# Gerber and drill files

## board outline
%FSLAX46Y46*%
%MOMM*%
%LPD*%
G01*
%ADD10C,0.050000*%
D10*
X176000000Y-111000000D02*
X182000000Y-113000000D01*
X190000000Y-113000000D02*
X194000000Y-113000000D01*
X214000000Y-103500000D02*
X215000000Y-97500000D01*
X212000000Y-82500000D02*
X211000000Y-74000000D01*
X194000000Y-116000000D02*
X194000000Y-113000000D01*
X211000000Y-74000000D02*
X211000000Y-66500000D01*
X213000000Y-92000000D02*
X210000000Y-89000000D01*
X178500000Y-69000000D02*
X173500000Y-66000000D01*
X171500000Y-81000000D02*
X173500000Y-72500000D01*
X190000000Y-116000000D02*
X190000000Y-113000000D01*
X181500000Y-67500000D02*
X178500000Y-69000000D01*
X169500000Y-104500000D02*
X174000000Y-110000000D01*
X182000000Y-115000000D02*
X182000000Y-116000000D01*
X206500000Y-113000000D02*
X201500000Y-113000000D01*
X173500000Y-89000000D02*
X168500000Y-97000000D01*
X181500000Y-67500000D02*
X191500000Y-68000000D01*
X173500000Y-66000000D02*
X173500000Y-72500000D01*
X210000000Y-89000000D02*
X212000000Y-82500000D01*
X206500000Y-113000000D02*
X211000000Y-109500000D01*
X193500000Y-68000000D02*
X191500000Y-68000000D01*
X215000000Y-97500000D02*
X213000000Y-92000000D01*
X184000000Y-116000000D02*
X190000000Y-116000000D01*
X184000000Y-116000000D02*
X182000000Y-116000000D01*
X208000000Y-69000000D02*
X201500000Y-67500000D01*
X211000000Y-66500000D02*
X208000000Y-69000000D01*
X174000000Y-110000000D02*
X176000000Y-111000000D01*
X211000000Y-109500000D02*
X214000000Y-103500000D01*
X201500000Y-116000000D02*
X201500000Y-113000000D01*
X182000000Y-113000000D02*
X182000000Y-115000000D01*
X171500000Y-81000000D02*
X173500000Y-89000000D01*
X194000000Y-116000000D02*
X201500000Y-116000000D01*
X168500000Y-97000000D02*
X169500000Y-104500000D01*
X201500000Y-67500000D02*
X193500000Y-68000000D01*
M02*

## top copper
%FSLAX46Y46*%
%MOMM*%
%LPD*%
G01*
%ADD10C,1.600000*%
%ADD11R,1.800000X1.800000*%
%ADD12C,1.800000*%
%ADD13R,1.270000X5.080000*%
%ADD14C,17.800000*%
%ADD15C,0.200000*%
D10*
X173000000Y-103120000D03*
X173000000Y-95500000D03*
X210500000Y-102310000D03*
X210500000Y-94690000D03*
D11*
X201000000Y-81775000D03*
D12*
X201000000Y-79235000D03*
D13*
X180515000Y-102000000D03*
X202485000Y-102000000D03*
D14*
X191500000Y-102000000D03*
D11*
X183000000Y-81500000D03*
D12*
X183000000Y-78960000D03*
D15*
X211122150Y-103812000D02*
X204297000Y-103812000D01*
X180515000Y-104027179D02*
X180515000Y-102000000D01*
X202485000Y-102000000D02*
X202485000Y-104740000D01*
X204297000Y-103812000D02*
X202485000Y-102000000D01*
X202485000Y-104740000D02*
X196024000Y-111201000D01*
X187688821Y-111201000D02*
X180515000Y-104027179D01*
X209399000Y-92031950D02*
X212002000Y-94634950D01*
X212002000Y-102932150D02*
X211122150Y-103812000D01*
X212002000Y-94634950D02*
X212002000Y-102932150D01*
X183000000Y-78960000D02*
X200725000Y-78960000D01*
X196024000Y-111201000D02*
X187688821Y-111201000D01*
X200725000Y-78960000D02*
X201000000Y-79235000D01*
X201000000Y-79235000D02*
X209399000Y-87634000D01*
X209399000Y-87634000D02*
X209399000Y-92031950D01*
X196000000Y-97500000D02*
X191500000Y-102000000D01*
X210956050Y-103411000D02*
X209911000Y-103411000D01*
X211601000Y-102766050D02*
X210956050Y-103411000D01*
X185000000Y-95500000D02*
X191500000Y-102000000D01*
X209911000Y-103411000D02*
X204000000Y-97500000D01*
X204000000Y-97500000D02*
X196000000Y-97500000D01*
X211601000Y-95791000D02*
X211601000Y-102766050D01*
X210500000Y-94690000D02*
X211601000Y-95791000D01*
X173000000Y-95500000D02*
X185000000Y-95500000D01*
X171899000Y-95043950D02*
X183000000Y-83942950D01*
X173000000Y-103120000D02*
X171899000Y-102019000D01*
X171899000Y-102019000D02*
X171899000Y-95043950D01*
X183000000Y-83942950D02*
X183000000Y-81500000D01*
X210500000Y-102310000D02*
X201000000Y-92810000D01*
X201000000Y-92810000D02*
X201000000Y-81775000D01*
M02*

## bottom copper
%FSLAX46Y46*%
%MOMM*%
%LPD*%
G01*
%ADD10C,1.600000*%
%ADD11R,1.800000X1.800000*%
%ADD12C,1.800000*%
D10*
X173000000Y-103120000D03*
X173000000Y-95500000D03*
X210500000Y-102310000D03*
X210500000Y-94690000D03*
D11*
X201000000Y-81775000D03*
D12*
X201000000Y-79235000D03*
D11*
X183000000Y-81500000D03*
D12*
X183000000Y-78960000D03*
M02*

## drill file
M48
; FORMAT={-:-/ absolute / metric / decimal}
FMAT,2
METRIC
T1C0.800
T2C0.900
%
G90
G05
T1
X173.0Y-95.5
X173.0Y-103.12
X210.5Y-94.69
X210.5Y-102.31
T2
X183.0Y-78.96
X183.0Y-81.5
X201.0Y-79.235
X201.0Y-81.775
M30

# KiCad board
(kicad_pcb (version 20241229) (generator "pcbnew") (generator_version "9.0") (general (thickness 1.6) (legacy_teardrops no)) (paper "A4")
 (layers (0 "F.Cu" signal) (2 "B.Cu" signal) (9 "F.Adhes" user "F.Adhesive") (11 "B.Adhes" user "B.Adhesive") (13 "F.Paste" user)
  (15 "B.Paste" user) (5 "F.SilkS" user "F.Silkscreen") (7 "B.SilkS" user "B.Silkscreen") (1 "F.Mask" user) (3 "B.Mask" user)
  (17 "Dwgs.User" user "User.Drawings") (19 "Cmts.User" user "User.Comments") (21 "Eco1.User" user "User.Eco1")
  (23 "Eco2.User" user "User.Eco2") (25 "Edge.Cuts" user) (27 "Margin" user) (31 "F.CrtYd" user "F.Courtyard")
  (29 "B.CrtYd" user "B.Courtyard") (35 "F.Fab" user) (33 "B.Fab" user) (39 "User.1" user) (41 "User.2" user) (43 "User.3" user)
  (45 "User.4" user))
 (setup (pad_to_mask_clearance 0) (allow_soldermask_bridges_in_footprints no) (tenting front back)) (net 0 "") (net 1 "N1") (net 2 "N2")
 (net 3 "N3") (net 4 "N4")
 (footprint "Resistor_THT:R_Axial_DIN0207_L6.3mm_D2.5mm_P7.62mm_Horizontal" (layer "F.Cu") (at 173 103.12 90)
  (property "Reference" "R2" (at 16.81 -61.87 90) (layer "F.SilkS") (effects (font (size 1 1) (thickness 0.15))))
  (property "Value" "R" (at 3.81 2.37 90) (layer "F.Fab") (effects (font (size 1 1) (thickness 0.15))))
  (pad "1" thru_hole circle (at 0 0 90) (size 1.6 1.6) (drill 0.8) (layers "*.Cu" "*.Mask") (remove_unused_layers no) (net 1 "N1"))
  (pad "2" thru_hole circle (at 7.62 0 90) (size 1.6 1.6) (drill 0.8) (layers "*.Cu" "*.Mask") (remove_unused_layers no) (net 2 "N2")))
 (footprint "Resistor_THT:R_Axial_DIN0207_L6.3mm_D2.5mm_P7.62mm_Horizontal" (layer "F.Cu") (at 210.5 102.31 90)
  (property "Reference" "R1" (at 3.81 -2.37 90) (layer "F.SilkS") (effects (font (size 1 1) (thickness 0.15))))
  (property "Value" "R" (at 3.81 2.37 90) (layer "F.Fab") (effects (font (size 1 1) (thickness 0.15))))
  (pad "1" thru_hole circle (at 0 0 90) (size 1.6 1.6) (drill 0.8) (layers "*.Cu" "*.Mask") (remove_unused_layers no) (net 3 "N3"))
  (pad "2" thru_hole circle (at 7.62 0 90) (size 1.6 1.6) (drill 0.8) (layers "*.Cu" "*.Mask") (remove_unused_layers no) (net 2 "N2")))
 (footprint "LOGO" (layer "F.Cu") (at 192 79)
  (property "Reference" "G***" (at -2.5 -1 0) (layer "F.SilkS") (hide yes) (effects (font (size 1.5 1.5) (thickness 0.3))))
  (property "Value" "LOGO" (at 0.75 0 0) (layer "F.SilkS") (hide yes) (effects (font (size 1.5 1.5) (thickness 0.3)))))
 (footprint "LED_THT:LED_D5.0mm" (layer "F.Cu") (at 201 81.775 90)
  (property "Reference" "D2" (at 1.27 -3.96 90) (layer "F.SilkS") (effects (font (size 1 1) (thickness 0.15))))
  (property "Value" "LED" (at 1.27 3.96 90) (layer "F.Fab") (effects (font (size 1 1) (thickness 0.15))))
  (pad "1" thru_hole rect (at 0 0 90) (size 1.8 1.8) (drill 0.9) (layers "*.Cu" "*.Mask") (remove_unused_layers no) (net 3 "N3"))
  (pad "2" thru_hole circle (at 2.54 0 90) (size 1.8 1.8) (drill 0.9) (layers "*.Cu" "*.Mask") (remove_unused_layers no) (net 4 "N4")))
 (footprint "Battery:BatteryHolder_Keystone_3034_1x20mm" (layer "F.Cu") (at 191.5 102)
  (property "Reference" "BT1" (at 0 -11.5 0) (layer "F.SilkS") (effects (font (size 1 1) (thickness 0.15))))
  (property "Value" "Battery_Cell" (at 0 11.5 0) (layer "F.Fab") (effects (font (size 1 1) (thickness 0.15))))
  (pad "1" smd rect (at -10.985 0) (size 1.27 5.08) (layers "F.Cu" "F.Mask" "F.Paste") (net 4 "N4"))
  (pad "1" smd rect (at 10.985 0) (size 1.27 5.08) (layers "F.Cu" "F.Mask" "F.Paste") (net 4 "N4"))
  (pad "2" smd circle (at 0 0) (size 17.8 17.8) (layers "F.Cu" "F.Mask") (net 2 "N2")))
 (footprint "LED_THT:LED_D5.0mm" (layer "F.Cu") (at 183 81.5 90)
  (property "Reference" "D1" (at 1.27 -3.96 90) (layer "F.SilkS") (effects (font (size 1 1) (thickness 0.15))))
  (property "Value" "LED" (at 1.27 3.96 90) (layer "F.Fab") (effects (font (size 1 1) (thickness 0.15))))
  (pad "1" thru_hole rect (at 0 0 90) (size 1.8 1.8) (drill 0.9) (layers "*.Cu" "*.Mask") (remove_unused_layers no) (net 1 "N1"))
  (pad "2" thru_hole circle (at 2.54 0 90) (size 1.8 1.8) (drill 0.9) (layers "*.Cu" "*.Mask") (remove_unused_layers no) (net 4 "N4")))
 (gr_line (start 176 111) (end 182 113) (stroke (width 0.05) (type default)) (layer "Edge.Cuts"))
 (gr_line (start 190 113) (end 194 113) (stroke (width 0.05) (type default)) (layer "Edge.Cuts"))
 (gr_line (start 214 103.5) (end 215 97.5) (stroke (width 0.05) (type default)) (layer "Edge.Cuts"))
 (gr_line (start 212 82.5) (end 211 74) (stroke (width 0.05) (type default)) (layer "Edge.Cuts"))
 (gr_line (start 194 116) (end 194 113) (stroke (width 0.05) (type default)) (layer "Edge.Cuts"))
 (gr_line (start 211 74) (end 211 66.5) (stroke (width 0.05) (type default)) (layer "Edge.Cuts"))
 (gr_line (start 213 92) (end 210 89) (stroke (width 0.05) (type default)) (layer "Edge.Cuts"))
 (gr_line (start 178.5 69) (end 173.5 66) (stroke (width 0.05) (type default)) (layer "Edge.Cuts"))
 (gr_line (start 171.5 81) (end 173.5 72.5) (stroke (width 0.05) (type default)) (layer "Edge.Cuts"))
 (gr_line (start 190 116) (end 190 113) (stroke (width 0.05) (type default)) (layer "Edge.Cuts"))
 (gr_line (start 181.5 67.5) (end 178.5 69) (stroke (width 0.05) (type default)) (layer "Edge.Cuts"))
 (gr_line (start 169.5 104.5) (end 174 110) (stroke (width 0.05) (type default)) (layer "Edge.Cuts"))
 (gr_line (start 182 115) (end 182 116) (stroke (width 0.05) (type default)) (layer "Edge.Cuts"))
 (gr_line (start 206.5 113) (end 201.5 113) (stroke (width 0.05) (type default)) (layer "Edge.Cuts"))
 (gr_line (start 173.5 89) (end 168.5 97) (stroke (width 0.05) (type default)) (layer "Edge.Cuts"))
 (gr_line (start 181.5 67.5) (end 191.5 68) (stroke (width 0.05) (type default)) (layer "Edge.Cuts"))
 (gr_line (start 173.5 66) (end 173.5 72.5) (stroke (width 0.05) (type default)) (layer "Edge.Cuts"))
 (gr_line (start 210 89) (end 212 82.5) (stroke (width 0.05) (type default)) (layer "Edge.Cuts"))
 (gr_line (start 206.5 113) (end 211 109.5) (stroke (width 0.05) (type default)) (layer "Edge.Cuts"))
 (gr_line (start 193.5 68) (end 191.5 68) (stroke (width 0.05) (type default)) (layer "Edge.Cuts"))
 (gr_line (start 215 97.5) (end 213 92) (stroke (width 0.05) (type default)) (layer "Edge.Cuts"))
 (gr_line (start 184 116) (end 190 116) (stroke (width 0.05) (type default)) (layer "Edge.Cuts"))
 (gr_line (start 184 116) (end 182 116) (stroke (width 0.05) (type default)) (layer "Edge.Cuts"))
 (gr_line (start 208 69) (end 201.5 67.5) (stroke (width 0.05) (type default)) (layer "Edge.Cuts"))
 (gr_line (start 211 66.5) (end 208 69) (stroke (width 0.05) (type default)) (layer "Edge.Cuts"))
 (gr_line (start 174 110) (end 176 111) (stroke (width 0.05) (type default)) (layer "Edge.Cuts"))
 (gr_line (start 211 109.5) (end 214 103.5) (stroke (width 0.05) (type default)) (layer "Edge.Cuts"))
 (gr_line (start 201.5 116) (end 201.5 113) (stroke (width 0.05) (type default)) (layer "Edge.Cuts"))
 (gr_line (start 182 113) (end 182 115) (stroke (width 0.05) (type default)) (layer "Edge.Cuts"))
 (gr_line (start 171.5 81) (end 173.5 89) (stroke (width 0.05) (type default)) (layer "Edge.Cuts"))
 (gr_line (start 194 116) (end 201.5 116) (stroke (width 0.05) (type default)) (layer "Edge.Cuts"))
 (gr_line (start 168.5 97) (end 169.5 104.5) (stroke (width 0.05) (type default)) (layer "Edge.Cuts"))
 (gr_line (start 201.5 67.5) (end 193.5 68) (stroke (width 0.05) (type default)) (layer "Edge.Cuts"))
 (segment (start 211.12215 103.812) (end 204.297 103.812) (width 0.2) (layer "F.Cu") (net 4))
 (segment (start 180.515 104.027179) (end 180.515 102) (width 0.2) (layer "F.Cu") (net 4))
 (segment (start 202.485 102) (end 202.485 104.74) (width 0.2) (layer "F.Cu") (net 4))
 (segment (start 204.297 103.812) (end 202.485 102) (width 0.2) (layer "F.Cu") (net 4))
 (segment (start 202.485 104.74) (end 196.024 111.201) (width 0.2) (layer "F.Cu") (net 4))
 (segment (start 187.688821 111.201) (end 180.515 104.027179) (width 0.2) (layer "F.Cu") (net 4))
 (segment (start 209.399 92.03195) (end 212.002 94.63495) (width 0.2) (layer "F.Cu") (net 4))
 (segment (start 212.002 102.93215) (end 211.12215 103.812) (width 0.2) (layer "F.Cu") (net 4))
 (segment (start 212.002 94.63495) (end 212.002 102.93215) (width 0.2) (layer "F.Cu") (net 4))
 (segment (start 183 78.96) (end 200.725 78.96) (width 0.2) (layer "F.Cu") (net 4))
 (segment (start 196.024 111.201) (end 187.688821 111.201) (width 0.2) (layer "F.Cu") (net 4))
 (segment (start 200.725 78.96) (end 201 79.235) (width 0.2) (layer "F.Cu") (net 4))
 (segment (start 201 79.235) (end 209.399 87.634) (width 0.2) (layer "F.Cu") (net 4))
 (segment (start 209.399 87.634) (end 209.399 92.03195) (width 0.2) (layer "F.Cu") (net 4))
 (segment (start 196 97.5) (end 191.5 102) (width 0.2) (layer "F.Cu") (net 2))
 (segment (start 210.95605 103.411) (end 209.911 103.411) (width 0.2) (layer "F.Cu") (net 2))
 (segment (start 211.601 102.76605) (end 210.95605 103.411) (width 0.2) (layer "F.Cu") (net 2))
 (segment (start 185 95.5) (end 191.5 102) (width 0.2) (layer "F.Cu") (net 2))
 (segment (start 209.911 103.411) (end 204 97.5) (width 0.2) (layer "F.Cu") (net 2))
 (segment (start 204 97.5) (end 196 97.5) (width 0.2) (layer "F.Cu") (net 2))
 (segment (start 211.601 95.791) (end 211.601 102.76605) (width 0.2) (layer "F.Cu") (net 2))
 (segment (start 210.5 94.69) (end 211.601 95.791) (width 0.2) (layer "F.Cu") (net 2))
 (segment (start 173 95.5) (end 185 95.5) (width 0.2) (layer "F.Cu") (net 2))
 (segment (start 171.899 95.04395) (end 183 83.94295) (width 0.2) (layer "F.Cu") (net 1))
 (segment (start 173 103.12) (end 171.899 102.019) (width 0.2) (layer "F.Cu") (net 1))
 (segment (start 171.899 102.019) (end 171.899 95.04395) (width 0.2) (layer "F.Cu") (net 1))
 (segment (start 183 83.94295) (end 183 81.5) (width 0.2) (layer "F.Cu") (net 1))
 (segment (start 210.5 102.31) (end 201 92.81) (width 0.2) (layer "F.Cu") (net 3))
 (segment (start 201 92.81) (end 201 81.775) (width 0.2) (layer "F.Cu") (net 3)))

